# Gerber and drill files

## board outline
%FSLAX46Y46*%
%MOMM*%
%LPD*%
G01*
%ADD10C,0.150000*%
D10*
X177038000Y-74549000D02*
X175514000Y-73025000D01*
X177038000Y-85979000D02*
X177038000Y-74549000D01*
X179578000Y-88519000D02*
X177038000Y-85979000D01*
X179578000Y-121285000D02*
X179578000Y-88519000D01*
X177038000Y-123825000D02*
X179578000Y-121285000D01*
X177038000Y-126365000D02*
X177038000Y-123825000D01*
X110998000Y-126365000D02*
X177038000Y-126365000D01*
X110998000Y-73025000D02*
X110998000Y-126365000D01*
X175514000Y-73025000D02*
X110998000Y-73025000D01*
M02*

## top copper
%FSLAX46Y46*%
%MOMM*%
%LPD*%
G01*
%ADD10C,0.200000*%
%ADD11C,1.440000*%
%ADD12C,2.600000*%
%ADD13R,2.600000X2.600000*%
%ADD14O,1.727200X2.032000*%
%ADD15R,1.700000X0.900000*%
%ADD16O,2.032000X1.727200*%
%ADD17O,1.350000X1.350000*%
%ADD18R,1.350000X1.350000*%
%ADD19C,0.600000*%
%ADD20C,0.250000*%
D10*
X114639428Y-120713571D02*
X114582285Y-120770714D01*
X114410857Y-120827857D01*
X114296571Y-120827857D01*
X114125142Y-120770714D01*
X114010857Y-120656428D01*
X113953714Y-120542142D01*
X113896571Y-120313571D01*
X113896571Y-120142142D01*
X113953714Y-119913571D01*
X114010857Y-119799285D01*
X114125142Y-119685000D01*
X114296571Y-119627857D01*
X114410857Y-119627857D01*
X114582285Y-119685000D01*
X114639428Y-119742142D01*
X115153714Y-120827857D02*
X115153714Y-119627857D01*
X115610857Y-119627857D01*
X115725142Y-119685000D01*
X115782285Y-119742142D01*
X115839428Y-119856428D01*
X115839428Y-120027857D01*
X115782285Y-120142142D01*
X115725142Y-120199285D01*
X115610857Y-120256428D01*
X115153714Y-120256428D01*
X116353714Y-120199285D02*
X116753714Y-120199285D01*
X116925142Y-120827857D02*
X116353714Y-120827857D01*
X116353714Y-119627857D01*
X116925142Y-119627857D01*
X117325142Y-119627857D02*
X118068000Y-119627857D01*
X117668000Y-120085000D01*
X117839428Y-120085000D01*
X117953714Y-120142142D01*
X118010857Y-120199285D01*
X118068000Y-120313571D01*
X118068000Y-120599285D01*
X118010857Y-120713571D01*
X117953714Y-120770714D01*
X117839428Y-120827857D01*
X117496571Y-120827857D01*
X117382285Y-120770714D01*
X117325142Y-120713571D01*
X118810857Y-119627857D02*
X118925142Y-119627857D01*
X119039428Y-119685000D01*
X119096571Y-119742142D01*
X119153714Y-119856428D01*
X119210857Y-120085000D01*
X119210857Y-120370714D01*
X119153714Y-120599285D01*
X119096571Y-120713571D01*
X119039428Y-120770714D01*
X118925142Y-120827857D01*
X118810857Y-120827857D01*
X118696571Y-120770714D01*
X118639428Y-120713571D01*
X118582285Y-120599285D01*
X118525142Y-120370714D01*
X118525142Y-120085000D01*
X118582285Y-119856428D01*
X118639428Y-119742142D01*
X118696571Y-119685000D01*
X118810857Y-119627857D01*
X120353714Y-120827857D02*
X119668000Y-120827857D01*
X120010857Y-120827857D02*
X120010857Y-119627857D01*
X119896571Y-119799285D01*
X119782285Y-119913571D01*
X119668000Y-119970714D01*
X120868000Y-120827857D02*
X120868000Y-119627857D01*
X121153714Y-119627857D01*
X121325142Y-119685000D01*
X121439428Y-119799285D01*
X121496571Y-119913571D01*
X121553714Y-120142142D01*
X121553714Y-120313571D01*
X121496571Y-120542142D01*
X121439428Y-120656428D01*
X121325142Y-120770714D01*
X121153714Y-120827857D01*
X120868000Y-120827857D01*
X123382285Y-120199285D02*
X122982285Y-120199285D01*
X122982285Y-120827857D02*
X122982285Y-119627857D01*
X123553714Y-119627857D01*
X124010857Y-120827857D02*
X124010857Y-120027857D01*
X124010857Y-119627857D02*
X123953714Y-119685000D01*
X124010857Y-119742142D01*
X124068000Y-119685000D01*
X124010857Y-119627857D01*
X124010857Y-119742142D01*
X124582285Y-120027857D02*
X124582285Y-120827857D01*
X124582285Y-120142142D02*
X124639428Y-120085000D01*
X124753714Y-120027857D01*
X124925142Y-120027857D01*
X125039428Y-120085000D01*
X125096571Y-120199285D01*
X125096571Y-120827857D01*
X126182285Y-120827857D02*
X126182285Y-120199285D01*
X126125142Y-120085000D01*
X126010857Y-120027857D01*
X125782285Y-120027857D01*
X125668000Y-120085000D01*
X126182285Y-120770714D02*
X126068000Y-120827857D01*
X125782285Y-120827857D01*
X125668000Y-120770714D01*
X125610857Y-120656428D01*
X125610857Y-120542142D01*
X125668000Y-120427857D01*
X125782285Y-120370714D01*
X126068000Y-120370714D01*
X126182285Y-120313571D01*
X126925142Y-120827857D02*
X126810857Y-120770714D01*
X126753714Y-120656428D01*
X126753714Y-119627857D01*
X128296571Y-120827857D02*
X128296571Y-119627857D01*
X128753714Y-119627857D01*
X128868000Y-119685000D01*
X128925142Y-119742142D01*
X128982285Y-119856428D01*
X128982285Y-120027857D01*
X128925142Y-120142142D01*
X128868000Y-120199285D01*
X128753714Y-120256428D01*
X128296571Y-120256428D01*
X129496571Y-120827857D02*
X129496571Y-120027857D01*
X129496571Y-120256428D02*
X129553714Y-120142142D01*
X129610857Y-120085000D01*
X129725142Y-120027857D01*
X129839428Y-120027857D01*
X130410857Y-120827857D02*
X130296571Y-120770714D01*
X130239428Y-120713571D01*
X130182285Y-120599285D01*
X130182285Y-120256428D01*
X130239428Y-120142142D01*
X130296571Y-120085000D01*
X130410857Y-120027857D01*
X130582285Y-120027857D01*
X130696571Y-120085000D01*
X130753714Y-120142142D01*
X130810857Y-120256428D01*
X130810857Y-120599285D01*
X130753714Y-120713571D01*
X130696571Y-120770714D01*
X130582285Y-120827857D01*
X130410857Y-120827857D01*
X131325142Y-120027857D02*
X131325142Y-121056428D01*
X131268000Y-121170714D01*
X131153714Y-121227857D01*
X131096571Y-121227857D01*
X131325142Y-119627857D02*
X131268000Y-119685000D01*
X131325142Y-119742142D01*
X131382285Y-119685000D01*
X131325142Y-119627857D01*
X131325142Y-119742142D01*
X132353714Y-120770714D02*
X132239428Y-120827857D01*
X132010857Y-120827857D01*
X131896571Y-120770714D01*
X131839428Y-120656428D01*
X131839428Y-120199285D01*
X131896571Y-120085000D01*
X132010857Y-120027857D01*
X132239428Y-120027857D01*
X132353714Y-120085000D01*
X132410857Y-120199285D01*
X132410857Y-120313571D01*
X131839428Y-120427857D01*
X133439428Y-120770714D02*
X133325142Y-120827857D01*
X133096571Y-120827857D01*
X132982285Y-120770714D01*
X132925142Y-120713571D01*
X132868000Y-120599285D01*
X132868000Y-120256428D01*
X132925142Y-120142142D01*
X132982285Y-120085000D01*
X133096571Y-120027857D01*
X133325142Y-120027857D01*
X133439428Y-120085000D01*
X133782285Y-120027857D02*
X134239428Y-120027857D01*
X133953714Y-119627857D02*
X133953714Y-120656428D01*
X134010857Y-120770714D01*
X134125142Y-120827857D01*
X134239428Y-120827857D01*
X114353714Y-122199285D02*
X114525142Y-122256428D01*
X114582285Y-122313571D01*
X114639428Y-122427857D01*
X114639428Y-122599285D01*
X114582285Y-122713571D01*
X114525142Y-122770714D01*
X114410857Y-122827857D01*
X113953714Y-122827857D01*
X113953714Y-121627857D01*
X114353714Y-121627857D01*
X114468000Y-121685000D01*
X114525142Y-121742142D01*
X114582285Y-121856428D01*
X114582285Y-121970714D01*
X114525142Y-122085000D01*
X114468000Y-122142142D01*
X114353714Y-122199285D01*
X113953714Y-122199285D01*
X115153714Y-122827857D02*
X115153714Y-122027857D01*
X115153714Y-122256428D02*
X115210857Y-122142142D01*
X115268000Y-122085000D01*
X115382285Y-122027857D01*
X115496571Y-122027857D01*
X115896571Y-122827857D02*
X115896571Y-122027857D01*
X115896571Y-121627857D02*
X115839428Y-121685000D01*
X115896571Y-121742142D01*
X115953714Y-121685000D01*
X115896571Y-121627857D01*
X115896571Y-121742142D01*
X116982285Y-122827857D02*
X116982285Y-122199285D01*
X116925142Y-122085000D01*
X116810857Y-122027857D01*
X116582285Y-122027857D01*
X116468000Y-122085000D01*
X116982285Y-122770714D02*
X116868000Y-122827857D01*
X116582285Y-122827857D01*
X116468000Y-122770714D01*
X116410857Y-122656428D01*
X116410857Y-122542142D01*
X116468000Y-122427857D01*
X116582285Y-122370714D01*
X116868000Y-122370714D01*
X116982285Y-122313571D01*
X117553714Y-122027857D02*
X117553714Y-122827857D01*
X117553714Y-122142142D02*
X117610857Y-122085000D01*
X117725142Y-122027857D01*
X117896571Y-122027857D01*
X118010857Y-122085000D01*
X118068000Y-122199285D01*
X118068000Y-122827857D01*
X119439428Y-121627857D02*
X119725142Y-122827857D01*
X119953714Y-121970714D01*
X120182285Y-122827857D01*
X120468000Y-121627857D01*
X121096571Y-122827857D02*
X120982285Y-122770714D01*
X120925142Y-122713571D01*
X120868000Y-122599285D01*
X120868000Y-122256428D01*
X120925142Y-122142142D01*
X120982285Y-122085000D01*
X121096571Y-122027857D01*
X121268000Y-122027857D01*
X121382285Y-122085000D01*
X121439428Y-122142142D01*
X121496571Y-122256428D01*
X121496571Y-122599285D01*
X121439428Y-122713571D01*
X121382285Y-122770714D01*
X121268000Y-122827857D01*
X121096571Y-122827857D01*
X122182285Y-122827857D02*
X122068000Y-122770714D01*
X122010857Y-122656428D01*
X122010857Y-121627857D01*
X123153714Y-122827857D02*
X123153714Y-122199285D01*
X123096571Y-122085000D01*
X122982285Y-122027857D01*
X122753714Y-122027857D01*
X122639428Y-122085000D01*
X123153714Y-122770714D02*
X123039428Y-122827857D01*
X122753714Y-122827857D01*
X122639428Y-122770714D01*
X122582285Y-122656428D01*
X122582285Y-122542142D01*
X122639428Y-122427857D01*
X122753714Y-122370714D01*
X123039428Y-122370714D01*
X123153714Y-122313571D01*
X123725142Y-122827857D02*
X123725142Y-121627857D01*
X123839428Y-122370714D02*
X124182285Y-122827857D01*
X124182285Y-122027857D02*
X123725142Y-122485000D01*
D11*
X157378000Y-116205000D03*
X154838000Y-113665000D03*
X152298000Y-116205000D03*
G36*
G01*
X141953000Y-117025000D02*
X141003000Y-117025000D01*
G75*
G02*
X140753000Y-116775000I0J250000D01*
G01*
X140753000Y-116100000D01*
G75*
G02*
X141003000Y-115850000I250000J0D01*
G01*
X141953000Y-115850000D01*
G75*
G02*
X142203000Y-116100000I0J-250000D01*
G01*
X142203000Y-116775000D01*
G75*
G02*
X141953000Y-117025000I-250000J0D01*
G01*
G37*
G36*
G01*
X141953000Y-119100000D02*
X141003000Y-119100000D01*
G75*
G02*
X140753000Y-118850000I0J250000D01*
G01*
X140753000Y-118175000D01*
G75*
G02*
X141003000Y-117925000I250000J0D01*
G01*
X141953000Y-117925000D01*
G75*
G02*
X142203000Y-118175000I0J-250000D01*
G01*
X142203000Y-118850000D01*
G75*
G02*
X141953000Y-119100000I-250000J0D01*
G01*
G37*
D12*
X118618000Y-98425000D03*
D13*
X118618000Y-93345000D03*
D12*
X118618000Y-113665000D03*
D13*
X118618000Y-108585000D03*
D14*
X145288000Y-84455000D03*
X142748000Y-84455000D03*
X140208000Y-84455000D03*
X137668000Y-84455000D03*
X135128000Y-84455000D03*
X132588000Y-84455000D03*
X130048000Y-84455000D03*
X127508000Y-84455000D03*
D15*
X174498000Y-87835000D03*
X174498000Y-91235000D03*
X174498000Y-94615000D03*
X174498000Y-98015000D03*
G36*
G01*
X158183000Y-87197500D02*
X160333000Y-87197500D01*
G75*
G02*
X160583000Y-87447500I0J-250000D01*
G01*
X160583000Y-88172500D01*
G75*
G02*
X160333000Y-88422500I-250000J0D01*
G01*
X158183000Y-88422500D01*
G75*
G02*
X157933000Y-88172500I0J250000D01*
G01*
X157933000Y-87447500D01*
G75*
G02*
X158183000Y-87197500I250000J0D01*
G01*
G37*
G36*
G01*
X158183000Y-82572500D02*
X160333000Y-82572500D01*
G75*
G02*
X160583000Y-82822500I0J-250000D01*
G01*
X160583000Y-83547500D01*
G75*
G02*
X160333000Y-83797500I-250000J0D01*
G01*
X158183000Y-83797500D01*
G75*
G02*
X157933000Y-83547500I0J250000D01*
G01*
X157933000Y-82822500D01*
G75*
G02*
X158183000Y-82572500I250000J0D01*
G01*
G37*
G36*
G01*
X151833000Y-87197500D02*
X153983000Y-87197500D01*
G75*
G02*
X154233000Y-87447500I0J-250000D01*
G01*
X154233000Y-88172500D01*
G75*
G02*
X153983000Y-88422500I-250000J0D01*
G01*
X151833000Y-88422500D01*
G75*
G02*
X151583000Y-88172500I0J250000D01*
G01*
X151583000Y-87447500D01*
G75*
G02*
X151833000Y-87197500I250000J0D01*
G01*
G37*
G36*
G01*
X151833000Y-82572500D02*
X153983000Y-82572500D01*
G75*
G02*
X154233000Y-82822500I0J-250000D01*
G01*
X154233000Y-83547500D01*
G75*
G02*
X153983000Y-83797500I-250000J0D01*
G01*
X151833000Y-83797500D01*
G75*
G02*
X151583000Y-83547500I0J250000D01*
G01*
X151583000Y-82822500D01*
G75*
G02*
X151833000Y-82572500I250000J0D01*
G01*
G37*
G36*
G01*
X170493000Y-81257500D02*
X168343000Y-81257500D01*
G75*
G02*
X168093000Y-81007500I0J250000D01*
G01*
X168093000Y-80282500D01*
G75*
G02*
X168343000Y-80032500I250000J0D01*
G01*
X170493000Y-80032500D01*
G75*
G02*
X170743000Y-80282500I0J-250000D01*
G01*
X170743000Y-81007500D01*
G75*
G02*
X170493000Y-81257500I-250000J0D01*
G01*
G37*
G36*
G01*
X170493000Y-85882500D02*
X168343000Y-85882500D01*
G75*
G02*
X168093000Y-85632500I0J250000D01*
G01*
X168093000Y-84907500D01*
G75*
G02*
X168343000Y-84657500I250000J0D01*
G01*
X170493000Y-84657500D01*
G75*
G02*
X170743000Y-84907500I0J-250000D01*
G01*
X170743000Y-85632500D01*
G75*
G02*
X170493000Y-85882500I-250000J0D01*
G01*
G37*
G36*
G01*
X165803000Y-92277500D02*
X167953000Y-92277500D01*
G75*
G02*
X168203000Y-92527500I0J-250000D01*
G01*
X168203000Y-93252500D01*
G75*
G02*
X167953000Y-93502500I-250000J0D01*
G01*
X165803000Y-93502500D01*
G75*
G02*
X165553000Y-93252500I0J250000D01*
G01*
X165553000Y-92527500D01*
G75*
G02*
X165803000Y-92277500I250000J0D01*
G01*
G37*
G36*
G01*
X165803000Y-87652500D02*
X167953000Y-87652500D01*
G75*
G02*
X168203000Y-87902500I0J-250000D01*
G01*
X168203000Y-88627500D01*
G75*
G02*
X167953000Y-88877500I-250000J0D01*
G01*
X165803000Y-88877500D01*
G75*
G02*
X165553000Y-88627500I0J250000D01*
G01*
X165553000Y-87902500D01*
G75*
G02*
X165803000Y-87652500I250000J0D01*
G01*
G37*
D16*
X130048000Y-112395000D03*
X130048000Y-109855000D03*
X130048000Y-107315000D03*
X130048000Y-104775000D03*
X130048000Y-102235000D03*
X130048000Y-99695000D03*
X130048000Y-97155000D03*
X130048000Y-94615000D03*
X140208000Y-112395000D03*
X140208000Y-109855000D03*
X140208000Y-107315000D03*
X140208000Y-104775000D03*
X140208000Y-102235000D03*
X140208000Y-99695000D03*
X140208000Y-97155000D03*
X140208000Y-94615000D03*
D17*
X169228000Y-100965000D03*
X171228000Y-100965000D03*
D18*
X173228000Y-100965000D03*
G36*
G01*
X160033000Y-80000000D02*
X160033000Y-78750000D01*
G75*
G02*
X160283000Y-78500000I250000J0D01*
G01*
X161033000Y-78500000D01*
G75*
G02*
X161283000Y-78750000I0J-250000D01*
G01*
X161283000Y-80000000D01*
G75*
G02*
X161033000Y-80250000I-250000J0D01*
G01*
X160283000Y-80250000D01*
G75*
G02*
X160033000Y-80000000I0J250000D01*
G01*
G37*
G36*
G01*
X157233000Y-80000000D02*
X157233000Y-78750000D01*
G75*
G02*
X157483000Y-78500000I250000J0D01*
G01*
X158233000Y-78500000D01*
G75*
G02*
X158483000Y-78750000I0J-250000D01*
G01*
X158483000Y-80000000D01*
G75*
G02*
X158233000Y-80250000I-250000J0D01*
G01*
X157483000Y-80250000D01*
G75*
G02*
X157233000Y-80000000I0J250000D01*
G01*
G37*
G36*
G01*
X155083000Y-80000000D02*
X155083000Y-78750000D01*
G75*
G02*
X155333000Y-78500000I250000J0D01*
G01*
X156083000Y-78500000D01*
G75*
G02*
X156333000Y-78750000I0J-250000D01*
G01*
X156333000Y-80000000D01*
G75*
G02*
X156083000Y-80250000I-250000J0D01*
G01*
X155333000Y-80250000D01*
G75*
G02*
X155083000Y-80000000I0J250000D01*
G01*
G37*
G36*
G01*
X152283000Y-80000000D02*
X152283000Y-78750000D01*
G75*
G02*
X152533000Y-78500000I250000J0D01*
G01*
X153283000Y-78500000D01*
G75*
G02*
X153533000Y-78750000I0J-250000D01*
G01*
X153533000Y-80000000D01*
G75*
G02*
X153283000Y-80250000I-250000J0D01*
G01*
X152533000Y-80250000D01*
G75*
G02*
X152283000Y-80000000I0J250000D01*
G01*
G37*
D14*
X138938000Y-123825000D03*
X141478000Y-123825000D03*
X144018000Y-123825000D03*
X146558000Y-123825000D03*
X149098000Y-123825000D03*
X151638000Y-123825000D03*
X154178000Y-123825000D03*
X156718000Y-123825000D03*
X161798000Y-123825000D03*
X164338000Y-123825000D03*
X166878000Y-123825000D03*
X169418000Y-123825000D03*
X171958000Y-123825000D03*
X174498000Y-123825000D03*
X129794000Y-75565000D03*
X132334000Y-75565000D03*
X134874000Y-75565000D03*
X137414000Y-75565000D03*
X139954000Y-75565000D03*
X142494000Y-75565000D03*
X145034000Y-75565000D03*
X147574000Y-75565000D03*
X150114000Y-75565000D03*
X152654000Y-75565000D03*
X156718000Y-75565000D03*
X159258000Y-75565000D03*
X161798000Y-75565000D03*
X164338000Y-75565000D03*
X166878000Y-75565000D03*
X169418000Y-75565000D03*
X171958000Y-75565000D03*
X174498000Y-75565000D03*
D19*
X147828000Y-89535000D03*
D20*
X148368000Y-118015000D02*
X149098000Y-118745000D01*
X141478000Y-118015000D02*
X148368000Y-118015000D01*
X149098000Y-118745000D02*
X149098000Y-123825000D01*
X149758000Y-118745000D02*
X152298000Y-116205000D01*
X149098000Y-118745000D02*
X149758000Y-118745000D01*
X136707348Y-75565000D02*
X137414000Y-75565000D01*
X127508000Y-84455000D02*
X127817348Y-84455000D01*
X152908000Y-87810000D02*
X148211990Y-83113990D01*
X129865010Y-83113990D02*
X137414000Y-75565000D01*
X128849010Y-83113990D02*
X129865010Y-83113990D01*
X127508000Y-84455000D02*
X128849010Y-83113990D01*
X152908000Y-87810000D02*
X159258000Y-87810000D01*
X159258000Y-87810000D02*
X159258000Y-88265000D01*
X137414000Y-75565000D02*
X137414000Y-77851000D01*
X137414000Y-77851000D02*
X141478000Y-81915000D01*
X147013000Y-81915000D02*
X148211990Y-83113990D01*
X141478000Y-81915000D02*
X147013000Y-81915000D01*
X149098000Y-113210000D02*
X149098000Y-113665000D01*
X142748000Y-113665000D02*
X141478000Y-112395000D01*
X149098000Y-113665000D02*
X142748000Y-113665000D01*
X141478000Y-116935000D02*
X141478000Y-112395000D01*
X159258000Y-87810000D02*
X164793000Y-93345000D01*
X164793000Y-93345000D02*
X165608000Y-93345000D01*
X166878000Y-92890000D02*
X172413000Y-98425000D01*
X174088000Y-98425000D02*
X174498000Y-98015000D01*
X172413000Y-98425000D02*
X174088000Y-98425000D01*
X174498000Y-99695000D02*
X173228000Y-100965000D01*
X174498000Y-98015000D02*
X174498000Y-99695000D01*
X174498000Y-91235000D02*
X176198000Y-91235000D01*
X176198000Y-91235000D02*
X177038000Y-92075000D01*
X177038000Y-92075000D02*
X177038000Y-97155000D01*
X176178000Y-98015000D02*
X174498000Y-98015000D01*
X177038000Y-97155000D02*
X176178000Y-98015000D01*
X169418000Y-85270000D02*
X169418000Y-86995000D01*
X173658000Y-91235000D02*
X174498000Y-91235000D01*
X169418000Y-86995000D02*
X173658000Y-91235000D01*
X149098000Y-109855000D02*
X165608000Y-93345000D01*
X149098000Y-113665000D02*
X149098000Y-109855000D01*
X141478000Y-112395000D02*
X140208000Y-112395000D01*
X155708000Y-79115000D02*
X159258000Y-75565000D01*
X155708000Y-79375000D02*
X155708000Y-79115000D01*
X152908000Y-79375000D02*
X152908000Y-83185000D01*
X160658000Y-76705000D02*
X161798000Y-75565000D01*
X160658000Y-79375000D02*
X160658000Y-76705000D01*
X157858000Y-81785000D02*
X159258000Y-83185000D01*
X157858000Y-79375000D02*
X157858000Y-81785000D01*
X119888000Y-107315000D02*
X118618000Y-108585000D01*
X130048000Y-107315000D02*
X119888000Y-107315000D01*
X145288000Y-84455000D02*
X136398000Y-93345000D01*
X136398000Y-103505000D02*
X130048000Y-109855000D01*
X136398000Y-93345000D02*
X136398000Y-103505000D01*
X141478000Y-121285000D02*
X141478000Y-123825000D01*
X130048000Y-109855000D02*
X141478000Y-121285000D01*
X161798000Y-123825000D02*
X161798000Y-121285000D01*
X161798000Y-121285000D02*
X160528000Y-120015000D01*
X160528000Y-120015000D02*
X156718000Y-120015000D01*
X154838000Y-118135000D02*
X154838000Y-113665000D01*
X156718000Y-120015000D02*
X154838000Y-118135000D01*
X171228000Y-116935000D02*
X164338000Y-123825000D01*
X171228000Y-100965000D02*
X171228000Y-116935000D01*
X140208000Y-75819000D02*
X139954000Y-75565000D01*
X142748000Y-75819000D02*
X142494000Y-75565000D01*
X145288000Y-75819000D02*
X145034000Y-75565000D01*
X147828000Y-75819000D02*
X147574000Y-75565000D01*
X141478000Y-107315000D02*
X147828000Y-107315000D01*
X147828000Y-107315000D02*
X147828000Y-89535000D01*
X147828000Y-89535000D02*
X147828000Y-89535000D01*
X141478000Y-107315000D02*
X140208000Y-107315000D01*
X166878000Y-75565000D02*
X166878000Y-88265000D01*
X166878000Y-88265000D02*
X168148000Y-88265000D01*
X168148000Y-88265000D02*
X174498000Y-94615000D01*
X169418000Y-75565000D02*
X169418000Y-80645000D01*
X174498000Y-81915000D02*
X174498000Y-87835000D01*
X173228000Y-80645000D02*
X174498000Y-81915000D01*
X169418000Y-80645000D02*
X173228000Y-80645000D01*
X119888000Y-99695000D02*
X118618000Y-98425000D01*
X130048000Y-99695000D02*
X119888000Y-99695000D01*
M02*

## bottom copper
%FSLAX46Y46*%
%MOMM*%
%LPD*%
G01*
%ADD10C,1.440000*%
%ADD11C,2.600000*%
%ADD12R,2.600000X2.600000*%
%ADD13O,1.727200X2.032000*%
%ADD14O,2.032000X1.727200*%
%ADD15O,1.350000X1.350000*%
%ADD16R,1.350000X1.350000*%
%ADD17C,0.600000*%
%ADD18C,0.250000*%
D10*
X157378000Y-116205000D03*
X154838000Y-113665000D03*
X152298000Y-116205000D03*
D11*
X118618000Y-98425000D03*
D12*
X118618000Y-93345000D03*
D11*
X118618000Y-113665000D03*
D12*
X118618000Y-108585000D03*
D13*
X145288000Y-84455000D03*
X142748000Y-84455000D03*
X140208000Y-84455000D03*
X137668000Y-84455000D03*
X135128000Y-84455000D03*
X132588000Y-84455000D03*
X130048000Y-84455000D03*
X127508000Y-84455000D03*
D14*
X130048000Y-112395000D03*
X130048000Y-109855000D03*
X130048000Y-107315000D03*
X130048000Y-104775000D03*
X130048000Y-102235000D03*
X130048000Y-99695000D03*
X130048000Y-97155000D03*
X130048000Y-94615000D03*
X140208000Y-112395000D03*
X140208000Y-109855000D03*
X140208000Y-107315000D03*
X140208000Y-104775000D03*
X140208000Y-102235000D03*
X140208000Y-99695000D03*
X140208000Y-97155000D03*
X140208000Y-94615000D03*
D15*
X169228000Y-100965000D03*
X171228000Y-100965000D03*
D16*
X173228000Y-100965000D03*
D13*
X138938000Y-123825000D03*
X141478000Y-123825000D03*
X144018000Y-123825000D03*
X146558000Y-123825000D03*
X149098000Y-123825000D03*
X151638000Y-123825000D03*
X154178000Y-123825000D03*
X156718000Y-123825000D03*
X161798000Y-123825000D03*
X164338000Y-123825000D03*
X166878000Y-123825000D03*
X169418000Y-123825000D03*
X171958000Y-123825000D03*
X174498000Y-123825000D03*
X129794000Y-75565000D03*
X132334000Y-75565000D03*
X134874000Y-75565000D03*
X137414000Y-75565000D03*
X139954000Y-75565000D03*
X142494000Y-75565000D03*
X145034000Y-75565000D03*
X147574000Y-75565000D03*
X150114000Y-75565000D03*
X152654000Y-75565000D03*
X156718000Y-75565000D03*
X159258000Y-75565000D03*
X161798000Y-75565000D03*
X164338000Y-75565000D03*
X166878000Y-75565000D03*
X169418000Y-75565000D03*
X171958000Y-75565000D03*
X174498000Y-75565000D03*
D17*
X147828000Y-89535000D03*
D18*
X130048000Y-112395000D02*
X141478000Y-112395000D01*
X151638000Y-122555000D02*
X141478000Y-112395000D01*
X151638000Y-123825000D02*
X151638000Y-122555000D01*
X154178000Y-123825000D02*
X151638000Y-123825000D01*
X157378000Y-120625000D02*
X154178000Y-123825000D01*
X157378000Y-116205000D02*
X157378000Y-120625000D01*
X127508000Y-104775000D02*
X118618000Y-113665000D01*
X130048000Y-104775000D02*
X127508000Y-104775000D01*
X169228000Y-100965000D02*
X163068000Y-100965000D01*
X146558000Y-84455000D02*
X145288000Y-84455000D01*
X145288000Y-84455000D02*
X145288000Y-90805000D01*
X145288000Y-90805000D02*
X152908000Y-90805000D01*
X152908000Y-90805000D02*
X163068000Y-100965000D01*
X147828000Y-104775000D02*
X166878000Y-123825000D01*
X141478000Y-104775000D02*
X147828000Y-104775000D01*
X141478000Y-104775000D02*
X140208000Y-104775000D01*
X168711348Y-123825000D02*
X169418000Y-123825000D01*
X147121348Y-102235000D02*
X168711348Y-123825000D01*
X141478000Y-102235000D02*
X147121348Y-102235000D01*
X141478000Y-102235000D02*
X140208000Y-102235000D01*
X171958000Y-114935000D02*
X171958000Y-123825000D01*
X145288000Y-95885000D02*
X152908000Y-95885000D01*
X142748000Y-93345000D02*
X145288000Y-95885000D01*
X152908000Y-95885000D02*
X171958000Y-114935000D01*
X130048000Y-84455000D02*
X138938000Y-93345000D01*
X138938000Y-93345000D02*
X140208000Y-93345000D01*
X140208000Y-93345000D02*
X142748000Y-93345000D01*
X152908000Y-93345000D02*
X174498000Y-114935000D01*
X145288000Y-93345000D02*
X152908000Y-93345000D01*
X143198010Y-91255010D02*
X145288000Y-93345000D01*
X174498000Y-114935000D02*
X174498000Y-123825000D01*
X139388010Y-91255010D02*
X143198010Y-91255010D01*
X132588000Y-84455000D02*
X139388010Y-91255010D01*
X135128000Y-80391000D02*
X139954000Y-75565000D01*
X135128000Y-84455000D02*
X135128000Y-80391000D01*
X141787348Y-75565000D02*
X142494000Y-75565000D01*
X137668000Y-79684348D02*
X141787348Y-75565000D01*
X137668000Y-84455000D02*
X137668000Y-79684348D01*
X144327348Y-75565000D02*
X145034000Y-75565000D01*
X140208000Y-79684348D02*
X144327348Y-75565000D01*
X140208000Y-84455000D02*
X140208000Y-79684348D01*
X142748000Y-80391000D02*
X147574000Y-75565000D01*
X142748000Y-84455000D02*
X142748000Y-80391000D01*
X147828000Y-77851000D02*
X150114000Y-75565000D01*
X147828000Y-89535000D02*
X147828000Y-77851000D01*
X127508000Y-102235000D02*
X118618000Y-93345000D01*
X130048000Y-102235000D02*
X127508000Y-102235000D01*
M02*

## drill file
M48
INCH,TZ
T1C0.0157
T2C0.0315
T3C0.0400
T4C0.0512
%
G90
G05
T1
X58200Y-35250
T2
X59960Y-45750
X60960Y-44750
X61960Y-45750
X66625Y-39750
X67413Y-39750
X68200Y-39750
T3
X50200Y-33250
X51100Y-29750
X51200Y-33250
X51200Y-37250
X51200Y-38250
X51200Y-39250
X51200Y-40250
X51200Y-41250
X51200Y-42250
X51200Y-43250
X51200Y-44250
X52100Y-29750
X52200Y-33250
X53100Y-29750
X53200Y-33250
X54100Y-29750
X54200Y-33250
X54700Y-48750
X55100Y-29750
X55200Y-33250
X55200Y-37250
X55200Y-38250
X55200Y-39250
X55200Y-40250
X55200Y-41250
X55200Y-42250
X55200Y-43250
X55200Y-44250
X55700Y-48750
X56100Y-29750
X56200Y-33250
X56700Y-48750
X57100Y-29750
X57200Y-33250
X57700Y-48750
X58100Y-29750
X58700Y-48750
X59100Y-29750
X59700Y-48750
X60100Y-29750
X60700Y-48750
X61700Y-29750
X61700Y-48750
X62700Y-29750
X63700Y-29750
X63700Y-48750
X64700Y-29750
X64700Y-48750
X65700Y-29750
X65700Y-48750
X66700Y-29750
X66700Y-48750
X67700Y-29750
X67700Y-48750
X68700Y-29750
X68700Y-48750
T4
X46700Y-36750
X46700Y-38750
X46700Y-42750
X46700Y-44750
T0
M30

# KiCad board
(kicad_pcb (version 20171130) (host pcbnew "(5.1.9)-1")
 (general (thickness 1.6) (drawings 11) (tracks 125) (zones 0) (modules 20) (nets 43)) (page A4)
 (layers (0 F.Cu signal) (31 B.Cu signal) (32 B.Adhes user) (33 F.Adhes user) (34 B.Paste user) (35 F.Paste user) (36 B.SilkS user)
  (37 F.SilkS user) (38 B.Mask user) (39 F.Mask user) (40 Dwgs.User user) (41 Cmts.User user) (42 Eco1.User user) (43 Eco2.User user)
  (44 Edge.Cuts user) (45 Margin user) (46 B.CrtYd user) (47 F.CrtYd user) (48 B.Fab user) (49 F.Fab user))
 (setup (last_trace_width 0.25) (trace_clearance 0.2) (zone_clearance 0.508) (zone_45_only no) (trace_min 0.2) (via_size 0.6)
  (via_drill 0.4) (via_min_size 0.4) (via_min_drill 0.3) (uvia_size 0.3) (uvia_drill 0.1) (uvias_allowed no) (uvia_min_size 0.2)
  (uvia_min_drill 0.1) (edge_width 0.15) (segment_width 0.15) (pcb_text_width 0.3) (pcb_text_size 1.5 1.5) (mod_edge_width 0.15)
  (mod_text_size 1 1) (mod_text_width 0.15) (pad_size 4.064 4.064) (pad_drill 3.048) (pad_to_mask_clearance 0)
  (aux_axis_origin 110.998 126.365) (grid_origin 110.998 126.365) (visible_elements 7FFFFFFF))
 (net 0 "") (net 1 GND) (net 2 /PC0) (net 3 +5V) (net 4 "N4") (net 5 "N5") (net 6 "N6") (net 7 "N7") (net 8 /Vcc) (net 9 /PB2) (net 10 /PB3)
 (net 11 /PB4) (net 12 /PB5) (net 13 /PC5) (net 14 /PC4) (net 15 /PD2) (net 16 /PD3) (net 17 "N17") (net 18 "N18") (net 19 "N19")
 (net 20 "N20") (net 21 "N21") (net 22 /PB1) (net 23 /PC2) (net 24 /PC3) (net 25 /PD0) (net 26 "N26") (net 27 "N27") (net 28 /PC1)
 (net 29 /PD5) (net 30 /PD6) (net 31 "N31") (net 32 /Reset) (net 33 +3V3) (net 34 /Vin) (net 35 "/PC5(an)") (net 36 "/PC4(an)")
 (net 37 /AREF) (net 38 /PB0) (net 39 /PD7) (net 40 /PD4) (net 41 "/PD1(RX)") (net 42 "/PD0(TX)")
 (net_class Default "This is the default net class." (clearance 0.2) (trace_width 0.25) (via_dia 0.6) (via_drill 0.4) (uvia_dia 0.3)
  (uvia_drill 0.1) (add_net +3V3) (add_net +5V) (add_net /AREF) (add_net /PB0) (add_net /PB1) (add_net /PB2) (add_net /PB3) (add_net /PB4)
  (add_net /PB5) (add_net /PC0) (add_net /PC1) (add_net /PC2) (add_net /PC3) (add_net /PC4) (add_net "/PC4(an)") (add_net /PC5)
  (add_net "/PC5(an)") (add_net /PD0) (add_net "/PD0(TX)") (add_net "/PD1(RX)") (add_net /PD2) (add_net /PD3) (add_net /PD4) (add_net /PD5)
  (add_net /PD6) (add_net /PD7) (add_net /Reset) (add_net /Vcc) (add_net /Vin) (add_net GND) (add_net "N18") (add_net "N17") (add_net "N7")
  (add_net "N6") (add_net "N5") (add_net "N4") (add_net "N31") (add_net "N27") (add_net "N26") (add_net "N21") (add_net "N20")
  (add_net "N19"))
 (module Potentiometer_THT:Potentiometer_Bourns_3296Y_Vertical (layer F.Cu) (at 152.298 116.205 180)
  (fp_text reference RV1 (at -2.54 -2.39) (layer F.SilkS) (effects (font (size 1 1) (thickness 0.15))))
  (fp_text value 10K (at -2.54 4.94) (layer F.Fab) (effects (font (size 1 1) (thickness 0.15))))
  (pad 3 thru_hole circle (at -5.08 0 180) (size 1.44 1.44) (drill 0.8) (layers *.Cu *.Mask) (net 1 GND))
  (pad 2 thru_hole circle (at -2.54 2.54 180) (size 1.44 1.44) (drill 0.8) (layers *.Cu *.Mask) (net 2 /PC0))
  (pad 1 thru_hole circle (at 0 0 180) (size 1.44 1.44) (drill 0.8) (layers *.Cu *.Mask) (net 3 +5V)))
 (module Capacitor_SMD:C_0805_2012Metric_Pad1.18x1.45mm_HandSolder (layer F.Cu) (at 141.478 117.475 90)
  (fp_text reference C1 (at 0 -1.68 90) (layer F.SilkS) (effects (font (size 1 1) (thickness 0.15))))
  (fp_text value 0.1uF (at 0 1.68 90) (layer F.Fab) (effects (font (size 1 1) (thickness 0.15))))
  (pad 2 smd roundrect (at 1.0375 0 90) (size 1.175 1.45) (layers F.Cu F.Paste F.Mask) (roundrect_rratio 0.2127659574468085) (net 1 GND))
  (pad 1 smd roundrect (at -1.0375 0 90) (size 1.175 1.45) (layers F.Cu F.Paste F.Mask) (roundrect_rratio 0.2127659574468085) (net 3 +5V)))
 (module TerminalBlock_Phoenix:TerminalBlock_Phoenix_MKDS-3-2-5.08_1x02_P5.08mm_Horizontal (layer F.Cu) (at 118.618 93.345 270)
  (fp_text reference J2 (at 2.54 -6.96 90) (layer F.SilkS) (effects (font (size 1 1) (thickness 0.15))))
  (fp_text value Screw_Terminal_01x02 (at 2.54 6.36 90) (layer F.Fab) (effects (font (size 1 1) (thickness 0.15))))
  (pad 2 thru_hole circle (at 5.08 0 270) (size 2.6 2.6) (drill 1.3) (layers *.Cu *.Mask) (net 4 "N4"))
  (pad 1 thru_hole rect (at 0 0 270) (size 2.6 2.6) (drill 1.3) (layers *.Cu *.Mask) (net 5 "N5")))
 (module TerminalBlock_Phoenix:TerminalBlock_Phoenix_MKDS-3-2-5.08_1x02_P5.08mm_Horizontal (layer F.Cu) (at 118.618 108.585 270)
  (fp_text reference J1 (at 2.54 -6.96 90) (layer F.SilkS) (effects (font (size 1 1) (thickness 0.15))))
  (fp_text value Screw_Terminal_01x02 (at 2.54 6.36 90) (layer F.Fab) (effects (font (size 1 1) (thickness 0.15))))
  (pad 2 thru_hole circle (at 5.08 0 270) (size 2.6 2.6) (drill 1.3) (layers *.Cu *.Mask) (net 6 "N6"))
  (pad 1 thru_hole rect (at 0 0 270) (size 2.6 2.6) (drill 1.3) (layers *.Cu *.Mask) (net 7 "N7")))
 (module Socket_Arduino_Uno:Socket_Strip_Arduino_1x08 (layer F.Cu) (at 127.508 84.455)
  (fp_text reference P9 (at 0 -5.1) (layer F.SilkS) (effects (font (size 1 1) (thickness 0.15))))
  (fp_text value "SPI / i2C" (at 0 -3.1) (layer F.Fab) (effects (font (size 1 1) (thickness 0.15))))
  (pad 8 thru_hole oval (at 17.78 0) (size 1.7272 2.032) (drill 1.016) (layers *.Cu *.Mask F.SilkS) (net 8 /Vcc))
  (pad 7 thru_hole oval (at 15.24 0) (size 1.7272 2.032) (drill 1.016) (layers *.Cu *.Mask F.SilkS) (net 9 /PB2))
  (pad 6 thru_hole oval (at 12.7 0) (size 1.7272 2.032) (drill 1.016) (layers *.Cu *.Mask F.SilkS) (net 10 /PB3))
  (pad 5 thru_hole oval (at 10.16 0) (size 1.7272 2.032) (drill 1.016) (layers *.Cu *.Mask F.SilkS) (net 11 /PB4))
  (pad 4 thru_hole oval (at 7.62 0) (size 1.7272 2.032) (drill 1.016) (layers *.Cu *.Mask F.SilkS) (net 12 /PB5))
  (pad 3 thru_hole oval (at 5.08 0) (size 1.7272 2.032) (drill 1.016) (layers *.Cu *.Mask F.SilkS) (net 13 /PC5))
  (pad 2 thru_hole oval (at 2.54 0) (size 1.7272 2.032) (drill 1.016) (layers *.Cu *.Mask F.SilkS) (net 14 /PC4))
  (pad 1 thru_hole oval (at 0 0) (size 1.7272 2.032) (drill 1.016) (layers *.Cu *.Mask F.SilkS) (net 1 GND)))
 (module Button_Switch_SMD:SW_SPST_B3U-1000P (layer F.Cu) (at 174.498 89.535 90)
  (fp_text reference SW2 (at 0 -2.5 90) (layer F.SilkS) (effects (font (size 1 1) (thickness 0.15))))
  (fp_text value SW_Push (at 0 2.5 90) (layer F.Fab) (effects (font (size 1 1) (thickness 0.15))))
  (pad 2 smd rect (at 1.7 0 90) (size 0.9 1.7) (layers F.Cu F.Paste F.Mask) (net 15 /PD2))
  (pad 1 smd rect (at -1.7 0 90) (size 0.9 1.7) (layers F.Cu F.Paste F.Mask) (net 1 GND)))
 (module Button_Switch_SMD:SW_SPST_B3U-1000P (layer F.Cu) (at 174.498 96.315 90)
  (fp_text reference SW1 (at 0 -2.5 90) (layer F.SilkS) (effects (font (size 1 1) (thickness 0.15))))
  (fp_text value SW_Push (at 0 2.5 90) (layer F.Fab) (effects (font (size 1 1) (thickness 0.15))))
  (pad 2 smd rect (at 1.7 0 90) (size 0.9 1.7) (layers F.Cu F.Paste F.Mask) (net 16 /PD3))
  (pad 1 smd rect (at -1.7 0 90) (size 0.9 1.7) (layers F.Cu F.Paste F.Mask) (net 1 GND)))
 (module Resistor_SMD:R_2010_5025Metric (layer F.Cu) (at 159.258 85.4975 270)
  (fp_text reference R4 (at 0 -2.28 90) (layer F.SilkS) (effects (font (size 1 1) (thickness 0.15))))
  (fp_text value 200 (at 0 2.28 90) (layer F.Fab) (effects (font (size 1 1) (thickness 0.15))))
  (pad 2 smd roundrect (at 2.3125 0 270) (size 1.225 2.65) (layers F.Cu F.Paste F.Mask) (roundrect_rratio 0.2040816326530612) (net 1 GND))
  (pad 1 smd roundrect (at -2.3125 0 270) (size 1.225 2.65) (layers F.Cu F.Paste F.Mask) (roundrect_rratio 0.2040816326530612)
   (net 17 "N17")))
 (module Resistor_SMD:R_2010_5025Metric (layer F.Cu) (at 152.908 85.4975 270)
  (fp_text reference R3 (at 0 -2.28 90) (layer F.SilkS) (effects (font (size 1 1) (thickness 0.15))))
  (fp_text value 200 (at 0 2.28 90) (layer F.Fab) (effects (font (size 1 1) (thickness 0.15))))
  (pad 2 smd roundrect (at 2.3125 0 270) (size 1.225 2.65) (layers F.Cu F.Paste F.Mask) (roundrect_rratio 0.2040816326530612) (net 1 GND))
  (pad 1 smd roundrect (at -2.3125 0 270) (size 1.225 2.65) (layers F.Cu F.Paste F.Mask) (roundrect_rratio 0.2040816326530612)
   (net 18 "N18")))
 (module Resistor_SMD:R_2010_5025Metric (layer F.Cu) (at 169.418 82.9575 90)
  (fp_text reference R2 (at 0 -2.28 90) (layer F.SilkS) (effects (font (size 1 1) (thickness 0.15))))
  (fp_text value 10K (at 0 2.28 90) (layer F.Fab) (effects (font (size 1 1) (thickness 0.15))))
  (pad 2 smd roundrect (at 2.3125 0 90) (size 1.225 2.65) (layers F.Cu F.Paste F.Mask) (roundrect_rratio 0.2040816326530612) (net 15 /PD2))
  (pad 1 smd roundrect (at -2.3125 0 90) (size 1.225 2.65) (layers F.Cu F.Paste F.Mask) (roundrect_rratio 0.2040816326530612) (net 1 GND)))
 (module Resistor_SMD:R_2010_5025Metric (layer F.Cu) (at 166.878 90.5775 270)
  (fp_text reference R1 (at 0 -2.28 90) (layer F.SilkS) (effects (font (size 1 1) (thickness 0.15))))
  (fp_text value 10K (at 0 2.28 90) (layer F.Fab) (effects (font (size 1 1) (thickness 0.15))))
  (pad 2 smd roundrect (at 2.3125 0 270) (size 1.225 2.65) (layers F.Cu F.Paste F.Mask) (roundrect_rratio 0.2040816326530612) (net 1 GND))
  (pad 1 smd roundrect (at -2.3125 0 270) (size 1.225 2.65) (layers F.Cu F.Paste F.Mask) (roundrect_rratio 0.2040816326530612) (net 16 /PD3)))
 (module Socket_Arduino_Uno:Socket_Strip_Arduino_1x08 (layer F.Cu) (at 130.048 94.615 270)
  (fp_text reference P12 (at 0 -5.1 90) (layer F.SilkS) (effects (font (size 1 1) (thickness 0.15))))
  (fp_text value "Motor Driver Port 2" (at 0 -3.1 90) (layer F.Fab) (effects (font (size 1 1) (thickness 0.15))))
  (pad 8 thru_hole oval (at 17.78 0 270) (size 1.7272 2.032) (drill 1.016) (layers *.Cu *.Mask F.SilkS) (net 1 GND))
  (pad 7 thru_hole oval (at 15.24 0 270) (size 1.7272 2.032) (drill 1.016) (layers *.Cu *.Mask F.SilkS) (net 8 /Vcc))
  (pad 6 thru_hole oval (at 12.7 0 270) (size 1.7272 2.032) (drill 1.016) (layers *.Cu *.Mask F.SilkS) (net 7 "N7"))
  (pad 5 thru_hole oval (at 10.16 0 270) (size 1.7272 2.032) (drill 1.016) (layers *.Cu *.Mask F.SilkS) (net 6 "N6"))
  (pad 4 thru_hole oval (at 7.62 0 270) (size 1.7272 2.032) (drill 1.016) (layers *.Cu *.Mask F.SilkS) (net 5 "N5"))
  (pad 3 thru_hole oval (at 5.08 0 270) (size 1.7272 2.032) (drill 1.016) (layers *.Cu *.Mask F.SilkS) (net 4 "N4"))
  (pad 2 thru_hole oval (at 2.54 0 270) (size 1.7272 2.032) (drill 1.016) (layers *.Cu *.Mask F.SilkS) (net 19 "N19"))
  (pad 1 thru_hole oval (at 0 0 270) (size 1.7272 2.032) (drill 1.016) (layers *.Cu *.Mask F.SilkS) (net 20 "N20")))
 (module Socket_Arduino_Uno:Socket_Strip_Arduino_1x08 (layer F.Cu) (at 140.208 94.615 270)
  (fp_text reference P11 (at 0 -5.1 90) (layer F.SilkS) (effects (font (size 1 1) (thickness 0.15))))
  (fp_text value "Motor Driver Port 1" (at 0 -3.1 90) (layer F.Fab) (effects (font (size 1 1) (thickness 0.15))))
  (pad 8 thru_hole oval (at 17.78 0 270) (size 1.7272 2.032) (drill 1.016) (layers *.Cu *.Mask F.SilkS) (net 1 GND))
  (pad 7 thru_hole oval (at 15.24 0 270) (size 1.7272 2.032) (drill 1.016) (layers *.Cu *.Mask F.SilkS) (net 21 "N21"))
  (pad 6 thru_hole oval (at 12.7 0 270) (size 1.7272 2.032) (drill 1.016) (layers *.Cu *.Mask F.SilkS) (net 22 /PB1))
  (pad 5 thru_hole oval (at 10.16 0 270) (size 1.7272 2.032) (drill 1.016) (layers *.Cu *.Mask F.SilkS) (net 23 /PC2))
  (pad 4 thru_hole oval (at 7.62 0 270) (size 1.7272 2.032) (drill 1.016) (layers *.Cu *.Mask F.SilkS) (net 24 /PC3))
  (pad 3 thru_hole oval (at 5.08 0 270) (size 1.7272 2.032) (drill 1.016) (layers *.Cu *.Mask F.SilkS) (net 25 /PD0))
  (pad 2 thru_hole oval (at 2.54 0 270) (size 1.7272 2.032) (drill 1.016) (layers *.Cu *.Mask F.SilkS) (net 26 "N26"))
  (pad 1 thru_hole oval (at 0 0 270) (size 1.7272 2.032) (drill 1.016) (layers *.Cu *.Mask F.SilkS) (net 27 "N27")))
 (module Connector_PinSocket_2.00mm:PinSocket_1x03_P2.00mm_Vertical (layer F.Cu) (at 173.228 100.965 270)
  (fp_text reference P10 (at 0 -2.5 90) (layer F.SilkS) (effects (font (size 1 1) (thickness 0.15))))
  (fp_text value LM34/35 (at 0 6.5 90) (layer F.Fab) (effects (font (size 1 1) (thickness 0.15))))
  (pad 3 thru_hole oval (at 0 4 270) (size 1.35 1.35) (drill 0.8) (layers *.Cu *.Mask) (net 8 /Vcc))
  (pad 2 thru_hole oval (at 0 2 270) (size 1.35 1.35) (drill 0.8) (layers *.Cu *.Mask) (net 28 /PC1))
  (pad 1 thru_hole rect (at 0 0 270) (size 1.35 1.35) (drill 0.8) (layers *.Cu *.Mask) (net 1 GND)))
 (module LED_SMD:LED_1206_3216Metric (layer F.Cu) (at 159.258 79.375)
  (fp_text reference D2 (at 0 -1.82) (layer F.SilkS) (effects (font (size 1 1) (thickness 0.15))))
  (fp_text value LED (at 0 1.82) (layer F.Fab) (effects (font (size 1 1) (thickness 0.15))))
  (pad 2 smd roundrect (at 1.4 0) (size 1.25 1.75) (layers F.Cu F.Paste F.Mask) (roundrect_rratio 0.2) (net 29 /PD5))
  (pad 1 smd roundrect (at -1.4 0) (size 1.25 1.75) (layers F.Cu F.Paste F.Mask) (roundrect_rratio 0.2) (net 17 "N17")))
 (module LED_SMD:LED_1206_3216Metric (layer F.Cu) (at 154.308 79.375)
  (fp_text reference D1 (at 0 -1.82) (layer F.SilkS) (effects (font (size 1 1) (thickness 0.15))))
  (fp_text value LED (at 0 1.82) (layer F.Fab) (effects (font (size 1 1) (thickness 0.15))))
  (pad 2 smd roundrect (at 1.4 0) (size 1.25 1.75) (layers F.Cu F.Paste F.Mask) (roundrect_rratio 0.2) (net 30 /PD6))
  (pad 1 smd roundrect (at -1.4 0) (size 1.25 1.75) (layers F.Cu F.Paste F.Mask) (roundrect_rratio 0.2) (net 18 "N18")))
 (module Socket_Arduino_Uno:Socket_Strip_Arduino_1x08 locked (layer F.Cu) (at 138.938 123.825)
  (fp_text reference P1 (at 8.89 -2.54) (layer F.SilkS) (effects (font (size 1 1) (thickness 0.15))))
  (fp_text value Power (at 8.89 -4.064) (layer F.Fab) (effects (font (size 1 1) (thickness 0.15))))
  (pad 1 thru_hole oval (at 0 0) (size 1.7272 2.032) (drill 1.016) (layers *.Cu *.Mask F.SilkS) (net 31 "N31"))
  (pad 2 thru_hole oval (at 2.54 0) (size 1.7272 2.032) (drill 1.016) (layers *.Cu *.Mask F.SilkS) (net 8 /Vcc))
  (pad 3 thru_hole oval (at 5.08 0) (size 1.7272 2.032) (drill 1.016) (layers *.Cu *.Mask F.SilkS) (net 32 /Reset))
  (pad 4 thru_hole oval (at 7.62 0) (size 1.7272 2.032) (drill 1.016) (layers *.Cu *.Mask F.SilkS) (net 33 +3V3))
  (pad 5 thru_hole oval (at 10.16 0) (size 1.7272 2.032) (drill 1.016) (layers *.Cu *.Mask F.SilkS) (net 3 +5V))
  (pad 6 thru_hole oval (at 12.7 0) (size 1.7272 2.032) (drill 1.016) (layers *.Cu *.Mask F.SilkS) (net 1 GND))
  (pad 7 thru_hole oval (at 15.24 0) (size 1.7272 2.032) (drill 1.016) (layers *.Cu *.Mask F.SilkS) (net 1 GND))
  (pad 8 thru_hole oval (at 17.78 0) (size 1.7272 2.032) (drill 1.016) (layers *.Cu *.Mask F.SilkS) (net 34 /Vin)))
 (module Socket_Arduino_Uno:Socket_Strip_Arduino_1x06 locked (layer F.Cu) (at 161.798 123.825)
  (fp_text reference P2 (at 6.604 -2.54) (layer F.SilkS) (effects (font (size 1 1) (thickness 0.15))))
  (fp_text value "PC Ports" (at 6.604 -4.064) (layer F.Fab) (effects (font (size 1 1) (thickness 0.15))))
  (pad 1 thru_hole oval (at 0 0) (size 1.7272 2.032) (drill 1.016) (layers *.Cu *.Mask F.SilkS) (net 2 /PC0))
  (pad 2 thru_hole oval (at 2.54 0) (size 1.7272 2.032) (drill 1.016) (layers *.Cu *.Mask F.SilkS) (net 28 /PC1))
  (pad 3 thru_hole oval (at 5.08 0) (size 1.7272 2.032) (drill 1.016) (layers *.Cu *.Mask F.SilkS) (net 23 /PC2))
  (pad 4 thru_hole oval (at 7.62 0) (size 1.7272 2.032) (drill 1.016) (layers *.Cu *.Mask F.SilkS) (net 24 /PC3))
  (pad 5 thru_hole oval (at 10.16 0) (size 1.7272 2.032) (drill 1.016) (layers *.Cu *.Mask F.SilkS) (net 14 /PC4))
  (pad 6 thru_hole oval (at 12.7 0) (size 1.7272 2.032) (drill 1.016) (layers *.Cu *.Mask F.SilkS) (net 13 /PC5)))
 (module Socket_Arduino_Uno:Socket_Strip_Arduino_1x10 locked (layer F.Cu) (at 129.794 75.565)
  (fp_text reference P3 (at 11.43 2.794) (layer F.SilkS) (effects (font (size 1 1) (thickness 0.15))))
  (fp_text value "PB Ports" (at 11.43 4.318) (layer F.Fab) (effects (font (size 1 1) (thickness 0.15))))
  (pad 1 thru_hole oval (at 0 0) (size 1.7272 2.032) (drill 1.016) (layers *.Cu *.Mask F.SilkS) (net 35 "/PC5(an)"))
  (pad 2 thru_hole oval (at 2.54 0) (size 1.7272 2.032) (drill 1.016) (layers *.Cu *.Mask F.SilkS) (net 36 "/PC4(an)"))
  (pad 3 thru_hole oval (at 5.08 0) (size 1.7272 2.032) (drill 1.016) (layers *.Cu *.Mask F.SilkS) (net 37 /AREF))
  (pad 4 thru_hole oval (at 7.62 0) (size 1.7272 2.032) (drill 1.016) (layers *.Cu *.Mask F.SilkS) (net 1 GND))
  (pad 5 thru_hole oval (at 10.16 0) (size 1.7272 2.032) (drill 1.016) (layers *.Cu *.Mask F.SilkS) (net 12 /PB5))
  (pad 6 thru_hole oval (at 12.7 0) (size 1.7272 2.032) (drill 1.016) (layers *.Cu *.Mask F.SilkS) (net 11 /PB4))
  (pad 7 thru_hole oval (at 15.24 0) (size 1.7272 2.032) (drill 1.016) (layers *.Cu *.Mask F.SilkS) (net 10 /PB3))
  (pad 8 thru_hole oval (at 17.78 0) (size 1.7272 2.032) (drill 1.016) (layers *.Cu *.Mask F.SilkS) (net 9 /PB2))
  (pad 9 thru_hole oval (at 20.32 0) (size 1.7272 2.032) (drill 1.016) (layers *.Cu *.Mask F.SilkS) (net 22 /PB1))
  (pad 10 thru_hole oval (at 22.86 0) (size 1.7272 2.032) (drill 1.016) (layers *.Cu *.Mask F.SilkS) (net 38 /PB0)))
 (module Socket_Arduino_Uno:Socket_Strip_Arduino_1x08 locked (layer F.Cu) (at 156.718 75.565)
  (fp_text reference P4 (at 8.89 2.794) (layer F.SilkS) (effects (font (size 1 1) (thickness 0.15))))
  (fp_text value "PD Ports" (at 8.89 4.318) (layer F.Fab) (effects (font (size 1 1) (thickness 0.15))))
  (pad 1 thru_hole oval (at 0 0) (size 1.7272 2.032) (drill 1.016) (layers *.Cu *.Mask F.SilkS) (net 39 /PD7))
  (pad 2 thru_hole oval (at 2.54 0) (size 1.7272 2.032) (drill 1.016) (layers *.Cu *.Mask F.SilkS) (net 30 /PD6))
  (pad 3 thru_hole oval (at 5.08 0) (size 1.7272 2.032) (drill 1.016) (layers *.Cu *.Mask F.SilkS) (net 29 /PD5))
  (pad 4 thru_hole oval (at 7.62 0) (size 1.7272 2.032) (drill 1.016) (layers *.Cu *.Mask F.SilkS) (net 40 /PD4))
  (pad 5 thru_hole oval (at 10.16 0) (size 1.7272 2.032) (drill 1.016) (layers *.Cu *.Mask F.SilkS) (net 16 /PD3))
  (pad 6 thru_hole oval (at 12.7 0) (size 1.7272 2.032) (drill 1.016) (layers *.Cu *.Mask F.SilkS) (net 15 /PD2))
  (pad 7 thru_hole oval (at 15.24 0) (size 1.7272 2.032) (drill 1.016) (layers *.Cu *.Mask F.SilkS) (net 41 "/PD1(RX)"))
  (pad 8 thru_hole oval (at 17.78 0) (size 1.7272 2.032) (drill 1.016) (layers *.Cu *.Mask F.SilkS) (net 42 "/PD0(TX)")))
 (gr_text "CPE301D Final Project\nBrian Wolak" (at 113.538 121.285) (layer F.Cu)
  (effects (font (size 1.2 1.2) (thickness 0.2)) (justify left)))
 (gr_line (start 177.038 74.549) (end 175.514 73.025) (angle 90) (layer Edge.Cuts) (width 0.15))
 (gr_line (start 177.038 85.979) (end 177.038 74.549) (angle 90) (layer Edge.Cuts) (width 0.15))
 (gr_line (start 179.578 88.519) (end 177.038 85.979) (angle 90) (layer Edge.Cuts) (width 0.15))
 (gr_line (start 179.578 121.285) (end 179.578 88.519) (angle 90) (layer Edge.Cuts) (width 0.15))
 (gr_line (start 177.038 123.825) (end 179.578 121.285) (angle 90) (layer Edge.Cuts) (width 0.15))
 (gr_line (start 177.038 126.365) (end 177.038 123.825) (angle 90) (layer Edge.Cuts) (width 0.15))
 (gr_line (start 110.998 126.365) (end 177.038 126.365) (angle 90) (layer Edge.Cuts) (width 0.15))
 (gr_line (start 110.998 73.025) (end 110.998 126.365) (angle 90) (layer Edge.Cuts) (width 0.15))
 (gr_line (start 175.514 73.025) (end 110.998 73.025) (angle 90) (layer Edge.Cuts) (width 0.15))
 (segment (start 148.368 118.015) (end 149.098 118.745) (width 0.25) (layer F.Cu) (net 3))
 (segment (start 141.478 118.015) (end 148.368 118.015) (width 0.25) (layer F.Cu) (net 3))
 (segment (start 149.098 118.745) (end 149.098 123.825) (width 0.25) (layer F.Cu) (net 3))
 (segment (start 149.758 118.745) (end 152.298 116.205) (width 0.25) (layer F.Cu) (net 3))
 (segment (start 149.098 118.745) (end 149.758 118.745) (width 0.25) (layer F.Cu) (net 3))
 (segment (start 136.707348 75.565) (end 137.414 75.565) (width 0.25) (layer F.Cu) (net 1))
 (segment (start 127.508 84.455) (end 127.817348 84.455) (width 0.25) (layer F.Cu) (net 1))
 (segment (start 152.908 87.81) (end 148.21199 83.11399) (width 0.25) (layer F.Cu) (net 1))
 (segment (start 129.86501 83.11399) (end 137.414 75.565) (width 0.25) (layer F.Cu) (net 1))
 (segment (start 128.84901 83.11399) (end 129.86501 83.11399) (width 0.25) (layer F.Cu) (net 1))
 (segment (start 127.508 84.455) (end 128.84901 83.11399) (width 0.25) (layer F.Cu) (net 1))
 (segment (start 152.908 87.81) (end 159.258 87.81) (width 0.25) (layer F.Cu) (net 1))
 (segment (start 159.258 87.81) (end 159.258 88.265) (width 0.25) (layer F.Cu) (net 1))
 (segment (start 137.414 75.565) (end 137.414 77.851) (width 0.25) (layer F.Cu) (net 1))
 (segment (start 137.414 77.851) (end 141.478 81.915) (width 0.25) (layer F.Cu) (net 1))
 (segment (start 147.013 81.915) (end 148.21199 83.11399) (width 0.25) (layer F.Cu) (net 1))
 (segment (start 141.478 81.915) (end 147.013 81.915) (width 0.25) (layer F.Cu) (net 1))
 (segment (start 130.048 112.395) (end 141.478 112.395) (width 0.25) (layer B.Cu) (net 1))
 (segment (start 149.098 113.21) (end 149.098 113.665) (width 0.25) (layer F.Cu) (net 1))
 (segment (start 142.748 113.665) (end 141.478 112.395) (width 0.25) (layer F.Cu) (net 1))
 (segment (start 149.098 113.665) (end 142.748 113.665) (width 0.25) (layer F.Cu) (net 1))
 (segment (start 141.478 116.935) (end 141.478 112.395) (width 0.25) (layer F.Cu) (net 1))
 (segment (start 151.638 122.555) (end 141.478 112.395) (width 0.25) (layer B.Cu) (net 1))
 (segment (start 151.638 123.825) (end 151.638 122.555) (width 0.25) (layer B.Cu) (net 1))
 (segment (start 154.178 123.825) (end 151.638 123.825) (width 0.25) (layer B.Cu) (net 1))
 (segment (start 159.258 87.81) (end 164.793 93.345) (width 0.25) (layer F.Cu) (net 1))
 (segment (start 164.793 93.345) (end 165.608 93.345) (width 0.25) (layer F.Cu) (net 1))
 (segment (start 166.878 92.89) (end 172.413 98.425) (width 0.25) (layer F.Cu) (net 1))
 (segment (start 174.088 98.425) (end 174.498 98.015) (width 0.25) (layer F.Cu) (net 1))
 (segment (start 172.413 98.425) (end 174.088 98.425) (width 0.25) (layer F.Cu) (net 1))
 (segment (start 174.498 99.695) (end 173.228 100.965) (width 0.25) (layer F.Cu) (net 1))
 (segment (start 174.498 98.015) (end 174.498 99.695) (width 0.25) (layer F.Cu) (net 1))
 (segment (start 174.498 91.235) (end 176.198 91.235) (width 0.25) (layer F.Cu) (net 1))
 (segment (start 176.198 91.235) (end 177.038 92.075) (width 0.25) (layer F.Cu) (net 1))
 (segment (start 177.038 92.075) (end 177.038 97.155) (width 0.25) (layer F.Cu) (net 1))
 (segment (start 176.178 98.015) (end 174.498 98.015) (width 0.25) (layer F.Cu) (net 1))
 (segment (start 177.038 97.155) (end 176.178 98.015) (width 0.25) (layer F.Cu) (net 1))
 (segment (start 169.418 85.27) (end 169.418 86.995) (width 0.25) (layer F.Cu) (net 1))
 (segment (start 173.658 91.235) (end 174.498 91.235) (width 0.25) (layer F.Cu) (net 1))
 (segment (start 169.418 86.995) (end 173.658 91.235) (width 0.25) (layer F.Cu) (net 1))
 (segment (start 149.098 109.855) (end 165.608 93.345) (width 0.25) (layer F.Cu) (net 1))
 (segment (start 149.098 113.665) (end 149.098 109.855) (width 0.25) (layer F.Cu) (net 1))
 (segment (start 157.378 120.625) (end 154.178 123.825) (width 0.25) (layer B.Cu) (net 1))
 (segment (start 157.378 116.205) (end 157.378 120.625) (width 0.25) (layer B.Cu) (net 1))
 (segment (start 141.478 112.395) (end 140.208 112.395) (width 0.25) (layer F.Cu) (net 1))
 (segment (start 155.708 79.115) (end 159.258 75.565) (width 0.25) (layer F.Cu) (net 30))
 (segment (start 155.708 79.375) (end 155.708 79.115) (width 0.25) (layer F.Cu) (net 30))
 (segment (start 152.908 79.375) (end 152.908 83.185) (width 0.25) (layer F.Cu) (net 18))
 (segment (start 160.658 76.705) (end 161.798 75.565) (width 0.25) (layer F.Cu) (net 29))
 (segment (start 160.658 79.375) (end 160.658 76.705) (width 0.25) (layer F.Cu) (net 29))
 (segment (start 157.858 81.785) (end 159.258 83.185) (width 0.25) (layer F.Cu) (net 17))
 (segment (start 157.858 79.375) (end 157.858 81.785) (width 0.25) (layer F.Cu) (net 17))
 (segment (start 127.508 104.775) (end 118.618 113.665) (width 0.25) (layer B.Cu) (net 6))
 (segment (start 130.048 104.775) (end 127.508 104.775) (width 0.25) (layer B.Cu) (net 6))
 (segment (start 119.888 107.315) (end 118.618 108.585) (width 0.25) (layer F.Cu) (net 7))
 (segment (start 130.048 107.315) (end 119.888 107.315) (width 0.25) (layer F.Cu) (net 7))
 (segment (start 169.228 100.965) (end 163.068 100.965) (width 0.25) (layer B.Cu) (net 8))
 (segment (start 146.558 84.455) (end 145.288 84.455) (width 0.25) (layer B.Cu) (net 8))
 (segment (start 145.288 84.455) (end 136.398 93.345) (width 0.25) (layer F.Cu) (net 8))
 (segment (start 136.398 103.505) (end 130.048 109.855) (width 0.25) (layer F.Cu) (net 8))
 (segment (start 136.398 93.345) (end 136.398 103.505) (width 0.25) (layer F.Cu) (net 8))
 (segment (start 141.478 121.285) (end 141.478 123.825) (width 0.25) (layer F.Cu) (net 8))
 (segment (start 130.048 109.855) (end 141.478 121.285) (width 0.25) (layer F.Cu) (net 8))
 (segment (start 145.288 84.455) (end 145.288 90.805) (width 0.25) (layer B.Cu) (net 8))
 (segment (start 145.288 90.805) (end 152.908 90.805) (width 0.25) (layer B.Cu) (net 8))
 (segment (start 152.908 90.805) (end 163.068 100.965) (width 0.25) (layer B.Cu) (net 8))
 (segment (start 161.798 123.825) (end 161.798 121.285) (width 0.25) (layer F.Cu) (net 2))
 (segment (start 161.798 121.285) (end 160.528 120.015) (width 0.25) (layer F.Cu) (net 2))
 (segment (start 160.528 120.015) (end 156.718 120.015) (width 0.25) (layer F.Cu) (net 2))
 (segment (start 154.838 118.135) (end 154.838 113.665) (width 0.25) (layer F.Cu) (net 2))
 (segment (start 156.718 120.015) (end 154.838 118.135) (width 0.25) (layer F.Cu) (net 2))
 (segment (start 171.228 116.935) (end 164.338 123.825) (width 0.25) (layer F.Cu) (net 28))
 (segment (start 171.228 100.965) (end 171.228 116.935) (width 0.25) (layer F.Cu) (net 28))
 (segment (start 147.828 104.775) (end 166.878 123.825) (width 0.25) (layer B.Cu) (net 23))
 (segment (start 141.478 104.775) (end 147.828 104.775) (width 0.25) (layer B.Cu) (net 23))
 (segment (start 141.478 104.775) (end 140.208 104.775) (width 0.25) (layer B.Cu) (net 23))
 (segment (start 168.711348 123.825) (end 169.418 123.825) (width 0.25) (layer B.Cu) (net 24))
 (segment (start 147.121348 102.235) (end 168.711348 123.825) (width 0.25) (layer B.Cu) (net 24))
 (segment (start 141.478 102.235) (end 147.121348 102.235) (width 0.25) (layer B.Cu) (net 24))
 (segment (start 141.478 102.235) (end 140.208 102.235) (width 0.25) (layer B.Cu) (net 24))
 (segment (start 171.958 114.935) (end 171.958 123.825) (width 0.25) (layer B.Cu) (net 14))
 (segment (start 145.288 95.885) (end 152.908 95.885) (width 0.25) (layer B.Cu) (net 14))
 (segment (start 142.748 93.345) (end 145.288 95.885) (width 0.25) (layer B.Cu) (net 14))
 (segment (start 152.908 95.885) (end 171.958 114.935) (width 0.25) (layer B.Cu) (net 14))
 (segment (start 130.048 84.455) (end 138.938 93.345) (width 0.25) (layer B.Cu) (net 14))
 (segment (start 138.938 93.345) (end 140.208 93.345) (width 0.25) (layer B.Cu) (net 14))
 (segment (start 140.208 93.345) (end 142.748 93.345) (width 0.25) (layer B.Cu) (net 14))
 (segment (start 152.908 93.345) (end 174.498 114.935) (width 0.25) (layer B.Cu) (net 13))
 (segment (start 145.288 93.345) (end 152.908 93.345) (width 0.25) (layer B.Cu) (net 13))
 (segment (start 143.19801 91.25501) (end 145.288 93.345) (width 0.25) (layer B.Cu) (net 13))
 (segment (start 174.498 114.935) (end 174.498 123.825) (width 0.25) (layer B.Cu) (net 13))
 (segment (start 139.38801 91.25501) (end 143.19801 91.25501) (width 0.25) (layer B.Cu) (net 13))
 (segment (start 132.588 84.455) (end 139.38801 91.25501) (width 0.25) (layer B.Cu) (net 13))
 (segment (start 140.208 75.819) (end 139.954 75.565) (width 0.25) (layer F.Cu) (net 12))
 (segment (start 135.128 80.391) (end 139.954 75.565) (width 0.25) (layer B.Cu) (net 12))
 (segment (start 135.128 84.455) (end 135.128 80.391) (width 0.25) (layer B.Cu) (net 12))
 (segment (start 142.748 75.819) (end 142.494 75.565) (width 0.25) (layer F.Cu) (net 11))
 (segment (start 141.787348 75.565) (end 142.494 75.565) (width 0.25) (layer B.Cu) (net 11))
 (segment (start 137.668 79.684348) (end 141.787348 75.565) (width 0.25) (layer B.Cu) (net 11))
 (segment (start 137.668 84.455) (end 137.668 79.684348) (width 0.25) (layer B.Cu) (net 11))
 (segment (start 145.288 75.819) (end 145.034 75.565) (width 0.25) (layer F.Cu) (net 10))
 (segment (start 144.327348 75.565) (end 145.034 75.565) (width 0.25) (layer B.Cu) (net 10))
 (segment (start 140.208 79.684348) (end 144.327348 75.565) (width 0.25) (layer B.Cu) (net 10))
 (segment (start 140.208 84.455) (end 140.208 79.684348) (width 0.25) (layer B.Cu) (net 10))
 (segment (start 147.828 75.819) (end 147.574 75.565) (width 0.25) (layer F.Cu) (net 9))
 (segment (start 142.748 80.391) (end 147.574 75.565) (width 0.25) (layer B.Cu) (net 9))
 (segment (start 142.748 84.455) (end 142.748 80.391) (width 0.25) (layer B.Cu) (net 9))
 (segment (start 141.478 107.315) (end 147.828 107.315) (width 0.25) (layer F.Cu) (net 22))
 (segment (start 147.828 107.315) (end 147.828 89.535) (width 0.25) (layer F.Cu) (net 22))
 (segment (start 147.828 89.535) (end 147.828 89.535) (width 0.25) (layer F.Cu) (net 22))
 (via (at 147.828 89.535) (size 0.6) (drill 0.4) (layers F.Cu B.Cu) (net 22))
 (segment (start 147.828 77.851) (end 150.114 75.565) (width 0.25) (layer B.Cu) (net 22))
 (segment (start 147.828 89.535) (end 147.828 77.851) (width 0.25) (layer B.Cu) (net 22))
 (segment (start 141.478 107.315) (end 140.208 107.315) (width 0.25) (layer F.Cu) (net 22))
 (segment (start 166.878 75.565) (end 166.878 88.265) (width 0.25) (layer F.Cu) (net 16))
 (segment (start 166.878 88.265) (end 168.148 88.265) (width 0.25) (layer F.Cu) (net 16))
 (segment (start 168.148 88.265) (end 174.498 94.615) (width 0.25) (layer F.Cu) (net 16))
 (segment (start 169.418 75.565) (end 169.418 80.645) (width 0.25) (layer F.Cu) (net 15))
 (segment (start 174.498 81.915) (end 174.498 87.835) (width 0.25) (layer F.Cu) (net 15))
 (segment (start 173.228 80.645) (end 174.498 81.915) (width 0.25) (layer F.Cu) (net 15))
 (segment (start 169.418 80.645) (end 173.228 80.645) (width 0.25) (layer F.Cu) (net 15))
 (segment (start 119.888 99.695) (end 118.618 98.425) (width 0.25) (layer F.Cu) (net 4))
 (segment (start 130.048 99.695) (end 119.888 99.695) (width 0.25) (layer F.Cu) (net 4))
 (segment (start 127.508 102.235) (end 118.618 93.345) (width 0.25) (layer B.Cu) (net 5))
 (segment (start 130.048 102.235) (end 127.508 102.235) (width 0.25) (layer B.Cu) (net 5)))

